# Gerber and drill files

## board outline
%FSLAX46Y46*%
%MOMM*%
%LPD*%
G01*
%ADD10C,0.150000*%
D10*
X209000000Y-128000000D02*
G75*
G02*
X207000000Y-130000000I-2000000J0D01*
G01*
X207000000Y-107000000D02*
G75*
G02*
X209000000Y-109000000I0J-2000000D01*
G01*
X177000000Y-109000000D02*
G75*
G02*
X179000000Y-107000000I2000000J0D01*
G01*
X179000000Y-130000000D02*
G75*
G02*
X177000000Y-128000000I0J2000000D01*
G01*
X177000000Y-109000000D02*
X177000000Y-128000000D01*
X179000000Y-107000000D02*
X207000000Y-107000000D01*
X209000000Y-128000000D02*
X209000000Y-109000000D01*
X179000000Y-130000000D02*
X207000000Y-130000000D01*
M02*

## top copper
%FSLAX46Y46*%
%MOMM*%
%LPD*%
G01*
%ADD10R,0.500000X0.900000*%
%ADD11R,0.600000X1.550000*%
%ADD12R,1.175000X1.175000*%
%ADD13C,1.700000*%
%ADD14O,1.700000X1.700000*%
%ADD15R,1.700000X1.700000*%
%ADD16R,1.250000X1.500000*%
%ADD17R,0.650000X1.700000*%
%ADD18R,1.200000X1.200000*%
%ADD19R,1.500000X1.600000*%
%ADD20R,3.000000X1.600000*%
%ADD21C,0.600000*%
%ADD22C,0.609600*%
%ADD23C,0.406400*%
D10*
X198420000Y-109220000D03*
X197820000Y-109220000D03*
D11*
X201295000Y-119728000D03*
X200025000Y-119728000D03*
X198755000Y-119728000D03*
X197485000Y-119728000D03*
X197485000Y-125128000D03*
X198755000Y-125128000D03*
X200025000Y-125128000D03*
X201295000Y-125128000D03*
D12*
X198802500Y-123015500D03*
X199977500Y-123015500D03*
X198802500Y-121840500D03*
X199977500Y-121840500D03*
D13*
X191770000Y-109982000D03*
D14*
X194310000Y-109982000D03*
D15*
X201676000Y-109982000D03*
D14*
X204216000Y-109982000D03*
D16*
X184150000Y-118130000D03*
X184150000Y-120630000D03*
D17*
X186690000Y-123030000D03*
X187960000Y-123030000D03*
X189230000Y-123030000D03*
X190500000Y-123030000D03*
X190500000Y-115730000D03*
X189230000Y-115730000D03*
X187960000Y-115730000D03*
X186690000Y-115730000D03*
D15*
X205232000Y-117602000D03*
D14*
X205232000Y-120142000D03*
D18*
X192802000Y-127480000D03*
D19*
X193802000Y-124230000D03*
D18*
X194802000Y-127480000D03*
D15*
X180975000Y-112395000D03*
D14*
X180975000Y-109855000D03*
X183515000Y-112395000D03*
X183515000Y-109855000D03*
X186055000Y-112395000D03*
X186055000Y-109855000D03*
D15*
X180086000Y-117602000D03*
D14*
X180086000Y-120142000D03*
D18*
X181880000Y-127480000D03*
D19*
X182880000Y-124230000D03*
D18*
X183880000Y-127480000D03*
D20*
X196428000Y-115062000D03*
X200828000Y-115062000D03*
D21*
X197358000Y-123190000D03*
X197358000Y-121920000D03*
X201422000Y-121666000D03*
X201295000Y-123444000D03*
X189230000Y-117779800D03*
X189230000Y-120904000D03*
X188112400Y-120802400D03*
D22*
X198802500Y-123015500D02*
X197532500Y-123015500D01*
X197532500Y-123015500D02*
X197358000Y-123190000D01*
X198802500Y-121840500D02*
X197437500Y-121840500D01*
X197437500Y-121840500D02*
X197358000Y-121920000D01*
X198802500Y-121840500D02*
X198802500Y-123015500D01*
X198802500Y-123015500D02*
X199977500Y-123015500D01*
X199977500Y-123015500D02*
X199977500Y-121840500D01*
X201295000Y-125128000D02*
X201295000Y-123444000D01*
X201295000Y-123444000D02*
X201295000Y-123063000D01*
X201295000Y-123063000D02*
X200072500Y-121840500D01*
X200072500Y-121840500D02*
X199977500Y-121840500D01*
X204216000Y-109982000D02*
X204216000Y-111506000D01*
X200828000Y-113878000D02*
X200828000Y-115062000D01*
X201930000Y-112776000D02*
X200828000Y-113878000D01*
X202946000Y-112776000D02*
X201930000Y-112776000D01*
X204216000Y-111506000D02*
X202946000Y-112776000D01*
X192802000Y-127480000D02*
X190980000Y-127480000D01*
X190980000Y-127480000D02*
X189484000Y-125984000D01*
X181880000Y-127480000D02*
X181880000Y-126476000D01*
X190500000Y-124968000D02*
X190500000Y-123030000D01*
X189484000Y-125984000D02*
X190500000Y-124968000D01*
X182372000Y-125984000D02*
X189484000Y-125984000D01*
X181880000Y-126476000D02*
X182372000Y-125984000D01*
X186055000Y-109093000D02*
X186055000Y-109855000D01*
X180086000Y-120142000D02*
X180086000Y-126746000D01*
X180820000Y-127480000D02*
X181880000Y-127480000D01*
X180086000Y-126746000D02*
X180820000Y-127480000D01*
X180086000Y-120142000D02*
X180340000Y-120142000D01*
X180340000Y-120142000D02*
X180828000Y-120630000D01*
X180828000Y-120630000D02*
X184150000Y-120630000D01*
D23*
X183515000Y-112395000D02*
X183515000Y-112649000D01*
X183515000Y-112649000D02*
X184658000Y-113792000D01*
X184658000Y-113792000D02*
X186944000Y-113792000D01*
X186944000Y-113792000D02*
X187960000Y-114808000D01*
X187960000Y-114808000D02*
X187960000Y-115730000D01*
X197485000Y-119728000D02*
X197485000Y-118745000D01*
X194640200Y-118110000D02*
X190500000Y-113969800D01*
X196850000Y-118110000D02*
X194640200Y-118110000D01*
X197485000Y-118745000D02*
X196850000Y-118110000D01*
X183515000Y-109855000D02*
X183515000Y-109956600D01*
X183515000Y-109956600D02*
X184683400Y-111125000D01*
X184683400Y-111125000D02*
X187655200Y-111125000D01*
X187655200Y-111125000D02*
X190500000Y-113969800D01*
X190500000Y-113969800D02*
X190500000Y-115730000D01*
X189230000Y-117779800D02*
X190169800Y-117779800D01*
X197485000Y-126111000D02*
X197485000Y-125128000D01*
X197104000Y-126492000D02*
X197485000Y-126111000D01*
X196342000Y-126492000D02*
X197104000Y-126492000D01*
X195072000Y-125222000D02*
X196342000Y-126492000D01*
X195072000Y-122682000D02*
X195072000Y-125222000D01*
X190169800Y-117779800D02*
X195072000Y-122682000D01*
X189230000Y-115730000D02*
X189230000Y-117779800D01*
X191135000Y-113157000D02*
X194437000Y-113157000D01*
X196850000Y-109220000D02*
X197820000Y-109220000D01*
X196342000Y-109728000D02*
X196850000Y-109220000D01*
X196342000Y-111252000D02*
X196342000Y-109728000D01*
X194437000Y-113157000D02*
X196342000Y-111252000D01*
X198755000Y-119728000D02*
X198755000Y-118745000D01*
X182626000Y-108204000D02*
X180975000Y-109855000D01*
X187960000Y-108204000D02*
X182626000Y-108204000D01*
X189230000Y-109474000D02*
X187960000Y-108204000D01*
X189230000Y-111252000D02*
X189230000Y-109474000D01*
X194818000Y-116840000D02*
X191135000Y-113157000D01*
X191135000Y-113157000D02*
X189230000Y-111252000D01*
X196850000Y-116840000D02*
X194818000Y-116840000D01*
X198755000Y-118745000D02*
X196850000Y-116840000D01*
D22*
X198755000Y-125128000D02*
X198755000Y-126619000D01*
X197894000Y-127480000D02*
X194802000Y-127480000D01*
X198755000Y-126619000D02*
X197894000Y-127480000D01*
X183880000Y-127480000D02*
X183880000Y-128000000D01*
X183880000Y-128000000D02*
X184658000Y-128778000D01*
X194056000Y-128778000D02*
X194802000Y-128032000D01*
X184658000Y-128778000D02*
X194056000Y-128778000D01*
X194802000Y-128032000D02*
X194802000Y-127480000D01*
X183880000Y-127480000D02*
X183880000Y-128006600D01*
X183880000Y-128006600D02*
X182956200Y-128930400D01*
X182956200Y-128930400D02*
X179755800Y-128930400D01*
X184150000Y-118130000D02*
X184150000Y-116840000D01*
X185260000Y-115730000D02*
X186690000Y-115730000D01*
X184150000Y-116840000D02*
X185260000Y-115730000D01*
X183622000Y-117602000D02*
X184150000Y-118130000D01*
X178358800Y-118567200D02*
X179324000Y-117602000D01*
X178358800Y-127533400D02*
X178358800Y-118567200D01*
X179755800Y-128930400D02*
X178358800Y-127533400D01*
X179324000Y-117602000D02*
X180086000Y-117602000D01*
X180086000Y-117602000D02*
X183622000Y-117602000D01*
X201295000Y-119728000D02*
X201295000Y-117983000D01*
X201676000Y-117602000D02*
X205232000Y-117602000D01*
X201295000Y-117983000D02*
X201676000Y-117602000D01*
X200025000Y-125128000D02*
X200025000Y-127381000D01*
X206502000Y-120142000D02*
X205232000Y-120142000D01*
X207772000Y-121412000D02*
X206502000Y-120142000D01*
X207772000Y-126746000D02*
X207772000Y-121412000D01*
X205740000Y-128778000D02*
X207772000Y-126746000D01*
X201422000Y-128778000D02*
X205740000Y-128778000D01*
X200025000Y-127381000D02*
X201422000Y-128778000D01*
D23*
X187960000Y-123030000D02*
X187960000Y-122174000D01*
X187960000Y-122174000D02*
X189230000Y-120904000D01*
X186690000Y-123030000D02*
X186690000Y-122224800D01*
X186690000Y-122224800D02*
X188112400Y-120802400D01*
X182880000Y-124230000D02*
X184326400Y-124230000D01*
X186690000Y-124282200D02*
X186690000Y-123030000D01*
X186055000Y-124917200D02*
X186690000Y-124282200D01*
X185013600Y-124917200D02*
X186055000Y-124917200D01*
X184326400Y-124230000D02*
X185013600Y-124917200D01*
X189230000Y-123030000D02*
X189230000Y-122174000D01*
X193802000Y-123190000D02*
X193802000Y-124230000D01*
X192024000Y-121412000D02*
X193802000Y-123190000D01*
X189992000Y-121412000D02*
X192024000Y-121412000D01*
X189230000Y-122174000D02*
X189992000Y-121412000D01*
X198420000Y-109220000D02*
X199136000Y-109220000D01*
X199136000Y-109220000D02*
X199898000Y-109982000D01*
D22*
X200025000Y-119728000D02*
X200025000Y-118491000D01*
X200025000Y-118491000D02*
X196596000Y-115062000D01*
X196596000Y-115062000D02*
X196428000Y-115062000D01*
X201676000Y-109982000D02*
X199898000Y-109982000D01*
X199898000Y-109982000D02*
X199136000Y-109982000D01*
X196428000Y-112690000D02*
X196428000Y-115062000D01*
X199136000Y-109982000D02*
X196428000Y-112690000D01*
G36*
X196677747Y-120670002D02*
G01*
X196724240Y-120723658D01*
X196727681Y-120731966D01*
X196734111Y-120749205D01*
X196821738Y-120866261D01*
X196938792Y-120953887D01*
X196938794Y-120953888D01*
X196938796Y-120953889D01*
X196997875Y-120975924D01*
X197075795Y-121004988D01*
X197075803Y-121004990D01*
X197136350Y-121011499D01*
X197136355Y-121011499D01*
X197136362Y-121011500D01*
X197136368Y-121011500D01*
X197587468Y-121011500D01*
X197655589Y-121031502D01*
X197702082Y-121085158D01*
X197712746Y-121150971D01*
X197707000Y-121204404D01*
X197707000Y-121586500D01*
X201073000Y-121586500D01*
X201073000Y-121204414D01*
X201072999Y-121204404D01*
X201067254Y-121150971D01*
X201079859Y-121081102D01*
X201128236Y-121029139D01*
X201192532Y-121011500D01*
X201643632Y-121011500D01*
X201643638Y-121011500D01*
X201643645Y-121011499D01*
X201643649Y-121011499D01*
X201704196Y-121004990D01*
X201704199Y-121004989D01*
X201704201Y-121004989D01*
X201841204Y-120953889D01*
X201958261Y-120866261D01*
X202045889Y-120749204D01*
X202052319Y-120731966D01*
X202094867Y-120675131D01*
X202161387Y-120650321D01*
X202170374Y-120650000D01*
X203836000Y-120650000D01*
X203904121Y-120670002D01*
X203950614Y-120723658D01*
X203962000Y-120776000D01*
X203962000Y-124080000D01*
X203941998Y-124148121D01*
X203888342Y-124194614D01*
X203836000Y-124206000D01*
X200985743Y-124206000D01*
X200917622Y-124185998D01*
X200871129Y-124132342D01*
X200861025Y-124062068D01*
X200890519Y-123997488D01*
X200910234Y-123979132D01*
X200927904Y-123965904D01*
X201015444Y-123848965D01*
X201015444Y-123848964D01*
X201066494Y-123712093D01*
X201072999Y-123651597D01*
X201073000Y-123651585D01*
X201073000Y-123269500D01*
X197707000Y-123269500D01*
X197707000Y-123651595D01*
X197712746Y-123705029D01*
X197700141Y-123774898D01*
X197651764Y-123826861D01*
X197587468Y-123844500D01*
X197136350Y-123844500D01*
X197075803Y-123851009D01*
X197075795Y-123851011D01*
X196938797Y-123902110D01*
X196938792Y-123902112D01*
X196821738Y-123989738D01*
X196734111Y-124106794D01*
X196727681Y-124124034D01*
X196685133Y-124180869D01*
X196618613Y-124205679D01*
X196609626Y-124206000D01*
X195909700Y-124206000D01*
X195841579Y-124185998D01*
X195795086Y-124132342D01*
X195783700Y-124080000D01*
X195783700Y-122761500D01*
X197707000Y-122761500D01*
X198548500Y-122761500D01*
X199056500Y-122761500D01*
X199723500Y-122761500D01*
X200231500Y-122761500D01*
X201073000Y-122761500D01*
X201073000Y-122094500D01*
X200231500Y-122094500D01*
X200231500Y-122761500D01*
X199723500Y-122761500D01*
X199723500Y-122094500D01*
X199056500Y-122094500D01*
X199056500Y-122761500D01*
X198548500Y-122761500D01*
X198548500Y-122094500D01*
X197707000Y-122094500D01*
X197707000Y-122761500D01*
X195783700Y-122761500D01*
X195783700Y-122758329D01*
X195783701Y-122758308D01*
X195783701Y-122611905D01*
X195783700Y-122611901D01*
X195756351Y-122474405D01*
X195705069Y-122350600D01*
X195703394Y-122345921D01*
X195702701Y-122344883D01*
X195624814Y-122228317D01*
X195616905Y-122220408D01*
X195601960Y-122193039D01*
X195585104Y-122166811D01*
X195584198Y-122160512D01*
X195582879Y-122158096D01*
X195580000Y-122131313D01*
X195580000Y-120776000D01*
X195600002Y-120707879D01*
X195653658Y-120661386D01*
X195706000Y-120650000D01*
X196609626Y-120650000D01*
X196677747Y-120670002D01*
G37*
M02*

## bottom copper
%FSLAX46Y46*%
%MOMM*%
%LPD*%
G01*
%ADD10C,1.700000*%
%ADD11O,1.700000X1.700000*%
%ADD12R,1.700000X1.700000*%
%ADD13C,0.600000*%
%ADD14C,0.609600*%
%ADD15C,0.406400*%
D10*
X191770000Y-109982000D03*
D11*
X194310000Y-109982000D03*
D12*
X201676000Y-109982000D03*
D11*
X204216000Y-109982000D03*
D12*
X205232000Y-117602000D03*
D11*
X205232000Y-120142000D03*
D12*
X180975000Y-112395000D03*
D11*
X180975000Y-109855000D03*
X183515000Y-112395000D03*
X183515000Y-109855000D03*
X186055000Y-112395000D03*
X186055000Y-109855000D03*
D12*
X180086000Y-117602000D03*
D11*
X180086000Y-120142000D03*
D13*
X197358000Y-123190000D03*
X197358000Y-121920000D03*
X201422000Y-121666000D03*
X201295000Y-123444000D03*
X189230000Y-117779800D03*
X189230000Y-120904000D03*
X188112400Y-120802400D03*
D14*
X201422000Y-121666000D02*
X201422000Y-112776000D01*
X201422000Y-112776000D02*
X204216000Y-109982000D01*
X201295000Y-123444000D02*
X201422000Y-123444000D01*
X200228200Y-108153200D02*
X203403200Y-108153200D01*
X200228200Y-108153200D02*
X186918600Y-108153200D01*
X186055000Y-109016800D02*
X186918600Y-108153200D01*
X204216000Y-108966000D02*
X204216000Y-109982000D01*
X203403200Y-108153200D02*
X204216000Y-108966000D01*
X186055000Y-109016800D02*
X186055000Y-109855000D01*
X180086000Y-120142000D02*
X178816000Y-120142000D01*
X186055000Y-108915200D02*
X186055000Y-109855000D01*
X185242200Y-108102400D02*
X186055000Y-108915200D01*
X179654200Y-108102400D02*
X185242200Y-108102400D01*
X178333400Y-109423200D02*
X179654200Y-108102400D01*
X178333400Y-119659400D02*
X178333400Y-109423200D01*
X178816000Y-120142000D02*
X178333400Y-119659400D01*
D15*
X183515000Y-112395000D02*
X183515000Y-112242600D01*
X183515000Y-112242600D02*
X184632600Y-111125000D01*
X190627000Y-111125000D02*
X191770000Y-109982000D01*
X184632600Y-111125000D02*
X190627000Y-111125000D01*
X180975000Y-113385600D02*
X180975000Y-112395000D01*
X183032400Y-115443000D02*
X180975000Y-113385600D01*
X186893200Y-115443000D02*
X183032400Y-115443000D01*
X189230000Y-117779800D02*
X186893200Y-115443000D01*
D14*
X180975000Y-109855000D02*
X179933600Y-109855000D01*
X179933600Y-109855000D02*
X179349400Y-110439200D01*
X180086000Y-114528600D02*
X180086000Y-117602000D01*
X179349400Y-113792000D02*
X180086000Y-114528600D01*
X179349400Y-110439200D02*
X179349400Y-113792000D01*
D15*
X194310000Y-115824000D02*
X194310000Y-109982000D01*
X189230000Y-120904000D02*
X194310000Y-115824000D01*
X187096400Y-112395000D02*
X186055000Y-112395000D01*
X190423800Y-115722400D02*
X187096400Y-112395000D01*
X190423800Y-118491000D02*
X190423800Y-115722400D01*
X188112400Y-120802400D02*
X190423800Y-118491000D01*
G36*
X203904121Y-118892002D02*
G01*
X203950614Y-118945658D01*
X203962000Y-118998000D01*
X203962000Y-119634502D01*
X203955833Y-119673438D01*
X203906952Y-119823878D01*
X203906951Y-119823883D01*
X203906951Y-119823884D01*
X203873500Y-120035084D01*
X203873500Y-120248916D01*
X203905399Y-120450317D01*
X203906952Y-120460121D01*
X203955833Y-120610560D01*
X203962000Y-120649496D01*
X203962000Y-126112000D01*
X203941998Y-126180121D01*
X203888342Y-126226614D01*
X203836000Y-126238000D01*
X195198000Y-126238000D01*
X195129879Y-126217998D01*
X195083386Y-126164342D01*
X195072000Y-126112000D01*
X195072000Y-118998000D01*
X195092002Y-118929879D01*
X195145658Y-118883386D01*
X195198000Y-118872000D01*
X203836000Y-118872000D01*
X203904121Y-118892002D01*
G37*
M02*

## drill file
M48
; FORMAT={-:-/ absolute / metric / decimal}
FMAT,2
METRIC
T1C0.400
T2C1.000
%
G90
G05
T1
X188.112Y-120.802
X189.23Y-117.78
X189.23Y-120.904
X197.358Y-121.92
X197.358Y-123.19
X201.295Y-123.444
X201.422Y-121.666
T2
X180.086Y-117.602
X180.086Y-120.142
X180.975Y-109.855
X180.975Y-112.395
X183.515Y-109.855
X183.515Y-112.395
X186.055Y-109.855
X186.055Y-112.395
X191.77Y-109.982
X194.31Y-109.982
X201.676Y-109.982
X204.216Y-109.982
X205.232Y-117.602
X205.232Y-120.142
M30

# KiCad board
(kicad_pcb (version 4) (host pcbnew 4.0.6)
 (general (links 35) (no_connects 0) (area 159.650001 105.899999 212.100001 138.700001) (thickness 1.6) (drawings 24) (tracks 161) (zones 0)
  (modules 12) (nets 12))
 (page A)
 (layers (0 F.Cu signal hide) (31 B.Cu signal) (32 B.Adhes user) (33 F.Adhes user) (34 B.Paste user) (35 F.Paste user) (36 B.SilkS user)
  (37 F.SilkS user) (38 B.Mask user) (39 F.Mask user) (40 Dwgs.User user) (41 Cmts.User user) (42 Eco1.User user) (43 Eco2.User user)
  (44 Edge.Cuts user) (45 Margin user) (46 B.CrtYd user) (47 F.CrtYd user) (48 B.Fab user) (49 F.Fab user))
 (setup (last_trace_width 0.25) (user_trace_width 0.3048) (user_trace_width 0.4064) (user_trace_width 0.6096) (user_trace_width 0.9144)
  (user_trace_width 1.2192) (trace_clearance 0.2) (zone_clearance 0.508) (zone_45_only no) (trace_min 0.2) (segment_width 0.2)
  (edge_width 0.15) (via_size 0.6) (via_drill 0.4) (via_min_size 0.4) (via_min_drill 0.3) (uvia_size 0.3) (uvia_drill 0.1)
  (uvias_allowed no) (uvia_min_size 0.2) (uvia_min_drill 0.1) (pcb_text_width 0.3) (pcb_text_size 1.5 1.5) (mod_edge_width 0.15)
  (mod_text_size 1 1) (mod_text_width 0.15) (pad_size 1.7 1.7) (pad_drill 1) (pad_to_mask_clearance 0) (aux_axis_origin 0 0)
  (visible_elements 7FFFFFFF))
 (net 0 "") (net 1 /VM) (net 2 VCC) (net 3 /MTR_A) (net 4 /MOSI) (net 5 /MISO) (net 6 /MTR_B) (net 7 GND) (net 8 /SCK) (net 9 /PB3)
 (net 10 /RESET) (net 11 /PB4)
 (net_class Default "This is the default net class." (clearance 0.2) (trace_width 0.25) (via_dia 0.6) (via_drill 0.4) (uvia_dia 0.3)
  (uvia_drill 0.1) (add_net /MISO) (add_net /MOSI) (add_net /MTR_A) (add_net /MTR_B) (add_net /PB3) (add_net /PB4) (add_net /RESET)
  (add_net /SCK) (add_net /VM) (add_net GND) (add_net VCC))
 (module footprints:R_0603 (layer F.Cu) (at 198.12 109.22 180)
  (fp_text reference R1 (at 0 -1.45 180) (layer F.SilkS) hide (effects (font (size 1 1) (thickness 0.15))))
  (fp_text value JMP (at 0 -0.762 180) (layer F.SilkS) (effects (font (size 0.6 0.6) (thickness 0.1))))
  (pad 1 smd rect (at -0.3 0 180) (size 0.5 0.9) (layers F.Cu F.Paste F.Mask) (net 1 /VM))
  (pad 2 smd rect (at 0.3 0 180) (size 0.5 0.9) (layers F.Cu F.Paste F.Mask) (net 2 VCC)))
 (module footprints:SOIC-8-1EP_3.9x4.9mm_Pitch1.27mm (layer F.Cu) (at 199.39 122.428 270)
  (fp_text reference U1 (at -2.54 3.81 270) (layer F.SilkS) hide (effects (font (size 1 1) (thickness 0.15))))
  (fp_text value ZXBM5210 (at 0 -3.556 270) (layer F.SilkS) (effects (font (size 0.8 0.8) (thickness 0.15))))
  (pad 1 smd rect (at -2.7 -1.905 270) (size 1.55 0.6) (layers F.Cu F.Paste F.Mask) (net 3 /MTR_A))
  (pad 2 smd rect (at -2.7 -0.635 270) (size 1.55 0.6) (layers F.Cu F.Paste F.Mask) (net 1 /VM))
  (pad 3 smd rect (at -2.7 0.635 270) (size 1.55 0.6) (layers F.Cu F.Paste F.Mask) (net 2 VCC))
  (pad 4 smd rect (at -2.7 1.905 270) (size 1.55 0.6) (layers F.Cu F.Paste F.Mask) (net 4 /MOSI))
  (pad 5 smd rect (at 2.7 1.905 270) (size 1.55 0.6) (layers F.Cu F.Paste F.Mask) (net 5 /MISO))
  (pad 6 smd rect (at 2.7 0.635 270) (size 1.55 0.6) (layers F.Cu F.Paste F.Mask) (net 2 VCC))
  (pad 7 smd rect (at 2.7 -0.635 270) (size 1.55 0.6) (layers F.Cu F.Paste F.Mask) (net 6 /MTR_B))
  (pad 8 smd rect (at 2.7 -1.905 270) (size 1.55 0.6) (layers F.Cu F.Paste F.Mask) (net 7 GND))
  (pad 8 smd rect (at 0.5875 0.5875 270) (size 1.175 1.175) (layers F.Cu F.Paste F.Mask) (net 7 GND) (solder_paste_margin_ratio -0.2))
  (pad 8 smd rect (at 0.5875 -0.5875 270) (size 1.175 1.175) (layers F.Cu F.Paste F.Mask) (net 7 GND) (solder_paste_margin_ratio -0.2))
  (pad 8 smd rect (at -0.5875 0.5875 270) (size 1.175 1.175) (layers F.Cu F.Paste F.Mask) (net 7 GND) (solder_paste_margin_ratio -0.2))
  (pad 8 smd rect (at -0.5875 -0.5875 270) (size 1.175 1.175) (layers F.Cu F.Paste F.Mask) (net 7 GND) (solder_paste_margin_ratio -0.2)))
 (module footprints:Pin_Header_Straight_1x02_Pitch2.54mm (layer F.Cu) (at 191.77 109.982 90)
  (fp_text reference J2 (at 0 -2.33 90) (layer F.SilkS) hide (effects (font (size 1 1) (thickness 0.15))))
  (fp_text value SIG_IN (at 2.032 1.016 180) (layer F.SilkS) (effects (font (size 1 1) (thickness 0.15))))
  (pad 1 thru_hole circle (at 0 0 90) (size 1.7 1.7) (drill 1) (layers *.Cu *.Mask) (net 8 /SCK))
  (pad 2 thru_hole oval (at 0 2.54 90) (size 1.7 1.7) (drill 1) (layers *.Cu *.Mask) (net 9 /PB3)))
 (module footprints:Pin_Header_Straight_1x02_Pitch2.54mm (layer F.Cu) (at 201.676 109.982 90)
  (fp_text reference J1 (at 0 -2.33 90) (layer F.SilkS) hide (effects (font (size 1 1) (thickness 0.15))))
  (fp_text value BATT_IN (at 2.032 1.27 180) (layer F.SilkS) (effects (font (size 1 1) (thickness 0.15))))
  (pad 1 thru_hole rect (at 0 0 90) (size 1.7 1.7) (drill 1) (layers *.Cu *.Mask) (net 1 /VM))
  (pad 2 thru_hole oval (at 0 2.54 90) (size 1.7 1.7) (drill 1) (layers *.Cu *.Mask) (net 7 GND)))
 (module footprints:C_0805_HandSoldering (layer F.Cu) (at 184.15 119.38 270)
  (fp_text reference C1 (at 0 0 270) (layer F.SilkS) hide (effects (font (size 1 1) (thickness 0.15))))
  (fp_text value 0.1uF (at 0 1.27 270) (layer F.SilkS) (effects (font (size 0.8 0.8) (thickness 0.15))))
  (pad 1 smd rect (at -1.25 0 270) (size 1.5 1.25) (layers F.Cu F.Paste F.Mask) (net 2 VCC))
  (pad 2 smd rect (at 1.25 0 270) (size 1.5 1.25) (layers F.Cu F.Paste F.Mask) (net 7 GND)))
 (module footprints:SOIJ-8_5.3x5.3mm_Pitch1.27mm (layer F.Cu) (at 188.595 119.38 90)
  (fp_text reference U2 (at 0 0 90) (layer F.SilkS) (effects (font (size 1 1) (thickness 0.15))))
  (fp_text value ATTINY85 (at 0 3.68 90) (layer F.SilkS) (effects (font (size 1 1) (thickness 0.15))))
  (pad 1 smd rect (at -3.65 -1.905 90) (size 1.7 0.65) (layers F.Cu F.Paste F.Mask) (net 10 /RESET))
  (pad 2 smd rect (at -3.65 -0.635 90) (size 1.7 0.65) (layers F.Cu F.Paste F.Mask) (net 9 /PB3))
  (pad 3 smd rect (at -3.65 0.635 90) (size 1.7 0.65) (layers F.Cu F.Paste F.Mask) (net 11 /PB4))
  (pad 4 smd rect (at -3.65 1.905 90) (size 1.7 0.65) (layers F.Cu F.Paste F.Mask) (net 7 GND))
  (pad 5 smd rect (at 3.65 1.905 90) (size 1.7 0.65) (layers F.Cu F.Paste F.Mask) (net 4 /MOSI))
  (pad 6 smd rect (at 3.65 0.635 90) (size 1.7 0.65) (layers F.Cu F.Paste F.Mask) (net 5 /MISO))
  (pad 7 smd rect (at 3.65 -0.635 90) (size 1.7 0.65) (layers F.Cu F.Paste F.Mask) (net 8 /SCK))
  (pad 8 smd rect (at 3.65 -1.905 90) (size 1.7 0.65) (layers F.Cu F.Paste F.Mask) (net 2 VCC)))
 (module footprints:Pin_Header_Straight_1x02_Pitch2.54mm (layer F.Cu) (at 205.232 117.602)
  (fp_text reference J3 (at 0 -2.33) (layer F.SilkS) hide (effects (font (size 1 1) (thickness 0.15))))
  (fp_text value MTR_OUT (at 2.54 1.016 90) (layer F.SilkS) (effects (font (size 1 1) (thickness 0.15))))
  (pad 1 thru_hole rect (at 0 0) (size 1.7 1.7) (drill 1) (layers *.Cu *.Mask) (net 3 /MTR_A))
  (pad 2 thru_hole oval (at 0 2.54) (size 1.7 1.7) (drill 1) (layers *.Cu *.Mask) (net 6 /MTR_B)))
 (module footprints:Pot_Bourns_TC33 (layer F.Cu) (at 193.802 125.73)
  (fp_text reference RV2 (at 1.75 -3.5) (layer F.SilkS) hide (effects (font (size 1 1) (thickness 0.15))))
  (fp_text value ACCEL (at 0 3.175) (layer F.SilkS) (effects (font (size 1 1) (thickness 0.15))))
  (pad 1 smd rect (at -1 1.75) (size 1.2 1.2) (layers F.Cu F.Mask) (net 7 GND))
  (pad 2 smd rect (at 0 -1.5) (size 1.5 1.6) (layers F.Cu F.Mask) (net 11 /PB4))
  (pad 3 smd rect (at 1 1.75) (size 1.2 1.2) (layers F.Cu F.Mask) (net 2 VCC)))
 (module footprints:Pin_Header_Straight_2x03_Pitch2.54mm (layer F.Cu) (at 180.975 112.395 90)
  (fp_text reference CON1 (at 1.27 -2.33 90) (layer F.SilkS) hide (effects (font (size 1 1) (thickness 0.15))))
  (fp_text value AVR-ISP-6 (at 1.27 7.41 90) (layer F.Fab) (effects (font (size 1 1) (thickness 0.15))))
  (pad 1 thru_hole rect (at 0 0 90) (size 1.7 1.7) (drill 1) (layers *.Cu *.Mask) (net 5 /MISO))
  (pad 2 thru_hole oval (at 2.54 0 90) (size 1.7 1.7) (drill 1) (layers *.Cu *.Mask) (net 2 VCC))
  (pad 3 thru_hole oval (at 0 2.54 90) (size 1.7 1.7) (drill 1) (layers *.Cu *.Mask) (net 8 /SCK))
  (pad 4 thru_hole oval (at 2.54 2.54 90) (size 1.7 1.7) (drill 1) (layers *.Cu *.Mask) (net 4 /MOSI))
  (pad 5 thru_hole oval (at 0 5.08 90) (size 1.7 1.7) (drill 1) (layers *.Cu *.Mask) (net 10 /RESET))
  (pad 6 thru_hole oval (at 2.54 5.08 90) (size 1.7 1.7) (drill 1) (layers *.Cu *.Mask) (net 7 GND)))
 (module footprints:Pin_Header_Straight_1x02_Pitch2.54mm (layer F.Cu) (at 180.086 117.602)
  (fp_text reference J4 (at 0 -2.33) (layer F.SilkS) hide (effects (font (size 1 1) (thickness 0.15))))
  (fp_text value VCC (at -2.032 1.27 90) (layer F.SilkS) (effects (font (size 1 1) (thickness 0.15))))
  (pad 1 thru_hole rect (at 0 0) (size 1.7 1.7) (drill 1) (layers *.Cu *.Mask) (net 2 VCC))
  (pad 2 thru_hole oval (at 0 2.54) (size 1.7 1.7) (drill 1) (layers *.Cu *.Mask) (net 7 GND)))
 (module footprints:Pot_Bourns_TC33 (layer F.Cu) (at 182.88 125.73)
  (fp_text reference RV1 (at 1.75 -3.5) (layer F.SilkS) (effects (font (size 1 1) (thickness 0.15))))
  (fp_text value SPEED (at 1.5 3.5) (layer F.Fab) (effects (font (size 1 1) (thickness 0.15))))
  (pad 1 smd rect (at -1 1.75) (size 1.2 1.2) (layers F.Cu F.Mask) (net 7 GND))
  (pad 2 smd rect (at 0 -1.5) (size 1.5 1.6) (layers F.Cu F.Mask) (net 10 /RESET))
  (pad 3 smd rect (at 1 1.75) (size 1.2 1.2) (layers F.Cu F.Mask) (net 2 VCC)))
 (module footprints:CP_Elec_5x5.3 (layer F.Cu) (at 198.628 115.062)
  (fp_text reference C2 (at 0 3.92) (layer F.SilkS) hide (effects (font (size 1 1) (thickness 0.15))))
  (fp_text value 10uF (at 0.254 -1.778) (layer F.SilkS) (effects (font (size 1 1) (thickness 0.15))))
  (pad 1 smd rect (at -2.2 0 180) (size 3 1.6) (layers F.Cu F.Paste F.Mask) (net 1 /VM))
  (pad 2 smd rect (at 2.2 0 180) (size 3 1.6) (layers F.Cu F.Paste F.Mask) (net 7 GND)))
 (gr_arc (start 207 128) (end 209 128) (angle 90) (layer Edge.Cuts) (width 0.15))
 (gr_arc (start 207 109) (end 207 107) (angle 90) (layer Edge.Cuts) (width 0.15))
 (gr_arc (start 179 109) (end 177 109) (angle 90) (layer Edge.Cuts) (width 0.15))
 (gr_arc (start 179 128) (end 179 130) (angle 90) (layer Edge.Cuts) (width 0.15))
 (gr_line (start 177 109) (end 177 128) (angle 90) (layer Edge.Cuts) (width 0.15))
 (gr_line (start 179 107) (end 207 107) (angle 90) (layer Edge.Cuts) (width 0.15))
 (gr_line (start 209 128) (end 209 109) (angle 90) (layer Edge.Cuts) (width 0.15))
 (gr_line (start 179 130) (end 207 130) (angle 90) (layer Edge.Cuts) (width 0.15))
 (segment (start 198.8025 123.0155) (end 197.5325 123.0155) (width 0.6096) (layer F.Cu) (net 7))
 (via (at 197.358 123.19) (size 0.6) (drill 0.4) (layers F.Cu B.Cu) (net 7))
 (segment (start 197.5325 123.0155) (end 197.358 123.19) (width 0.6096) (layer F.Cu) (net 7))
 (segment (start 198.8025 121.8405) (end 197.4375 121.8405) (width 0.6096) (layer F.Cu) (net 7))
 (via (at 197.358 121.92) (size 0.6) (drill 0.4) (layers F.Cu B.Cu) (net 7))
 (segment (start 197.4375 121.8405) (end 197.358 121.92) (width 0.6096) (layer F.Cu) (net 7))
 (segment (start 201.422 121.666) (end 201.422 112.776) (width 0.6096) (layer B.Cu) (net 7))
 (via (at 201.422 121.666) (size 0.6) (drill 0.4) (layers F.Cu B.Cu) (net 7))
 (segment (start 201.422 112.776) (end 204.216 109.982) (width 0.6096) (layer B.Cu) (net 7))
 (via (at 201.295 123.444) (size 0.6) (drill 0.4) (layers F.Cu B.Cu) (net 7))
 (segment (start 201.295 123.444) (end 201.422 123.444) (width 0.6096) (layer B.Cu) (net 7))
 (segment (start 198.8025 121.8405) (end 198.8025 123.0155) (width 0.6096) (layer F.Cu) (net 7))
 (segment (start 198.8025 123.0155) (end 199.9775 123.0155) (width 0.6096) (layer F.Cu) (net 7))
 (segment (start 199.9775 123.0155) (end 199.9775 121.8405) (width 0.6096) (layer F.Cu) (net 7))
 (segment (start 201.295 125.128) (end 201.295 123.444) (width 0.6096) (layer F.Cu) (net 7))
 (segment (start 201.295 123.444) (end 201.295 123.063) (width 0.6096) (layer F.Cu) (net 7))
 (segment (start 201.295 123.063) (end 200.0725 121.8405) (width 0.6096) (layer F.Cu) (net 7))
 (segment (start 200.0725 121.8405) (end 199.9775 121.8405) (width 0.6096) (layer F.Cu) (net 7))
 (segment (start 204.216 109.982) (end 204.216 111.506) (width 0.6096) (layer F.Cu) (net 7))
 (segment (start 200.828 113.878) (end 200.828 115.062) (width 0.6096) (layer F.Cu) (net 7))
 (segment (start 201.93 112.776) (end 200.828 113.878) (width 0.6096) (layer F.Cu) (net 7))
 (segment (start 202.946 112.776) (end 201.93 112.776) (width 0.6096) (layer F.Cu) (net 7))
 (segment (start 204.216 111.506) (end 202.946 112.776) (width 0.6096) (layer F.Cu) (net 7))
 (segment (start 192.802 127.48) (end 190.98 127.48) (width 0.6096) (layer F.Cu) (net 7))
 (segment (start 190.98 127.48) (end 189.484 125.984) (width 0.6096) (layer F.Cu) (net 7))
 (segment (start 200.2282 108.1532) (end 203.4032 108.1532) (width 0.6096) (layer B.Cu) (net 7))
 (segment (start 200.2282 108.1532) (end 186.9186 108.1532) (width 0.6096) (layer B.Cu) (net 7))
 (segment (start 186.055 109.0168) (end 186.9186 108.1532) (width 0.6096) (layer B.Cu) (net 7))
 (segment (start 204.216 108.966) (end 204.216 109.982) (width 0.6096) (layer B.Cu) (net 7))
 (segment (start 203.4032 108.1532) (end 204.216 108.966) (width 0.6096) (layer B.Cu) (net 7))
 (segment (start 186.055 109.0168) (end 186.055 109.855) (width 0.6096) (layer B.Cu) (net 7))
 (segment (start 180.086 120.142) (end 178.816 120.142) (width 0.6096) (layer B.Cu) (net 7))
 (segment (start 186.055 108.9152) (end 186.055 109.855) (width 0.6096) (layer B.Cu) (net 7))
 (segment (start 185.2422 108.1024) (end 186.055 108.9152) (width 0.6096) (layer B.Cu) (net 7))
 (segment (start 179.6542 108.1024) (end 185.2422 108.1024) (width 0.6096) (layer B.Cu) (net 7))
 (segment (start 178.3334 109.4232) (end 179.6542 108.1024) (width 0.6096) (layer B.Cu) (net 7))
 (segment (start 178.3334 119.6594) (end 178.3334 109.4232) (width 0.6096) (layer B.Cu) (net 7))
 (segment (start 178.816 120.142) (end 178.3334 119.6594) (width 0.6096) (layer B.Cu) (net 7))
 (segment (start 181.88 127.48) (end 181.88 126.476) (width 0.6096) (layer F.Cu) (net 7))
 (segment (start 190.5 124.968) (end 190.5 123.03) (width 0.6096) (layer F.Cu) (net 7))
 (segment (start 189.484 125.984) (end 190.5 124.968) (width 0.6096) (layer F.Cu) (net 7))
 (segment (start 182.372 125.984) (end 189.484 125.984) (width 0.6096) (layer F.Cu) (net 7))
 (segment (start 181.88 126.476) (end 182.372 125.984) (width 0.6096) (layer F.Cu) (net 7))
 (segment (start 186.055 109.093) (end 186.055 109.855) (width 0.6096) (layer F.Cu) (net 7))
 (segment (start 180.086 120.142) (end 180.086 126.746) (width 0.6096) (layer F.Cu) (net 7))
 (segment (start 180.82 127.48) (end 181.88 127.48) (width 0.6096) (layer F.Cu) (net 7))
 (segment (start 180.086 126.746) (end 180.82 127.48) (width 0.6096) (layer F.Cu) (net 7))
 (segment (start 180.086 120.142) (end 180.34 120.142) (width 0.6096) (layer F.Cu) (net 7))
 (segment (start 180.34 120.142) (end 180.828 120.63) (width 0.6096) (layer F.Cu) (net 7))
 (segment (start 180.828 120.63) (end 184.15 120.63) (width 0.6096) (layer F.Cu) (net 7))
 (segment (start 183.515 112.395) (end 183.515 112.2426) (width 0.4064) (layer B.Cu) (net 8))
 (segment (start 183.515 112.2426) (end 184.6326 111.125) (width 0.4064) (layer B.Cu) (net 8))
 (segment (start 190.627 111.125) (end 191.77 109.982) (width 0.4064) (layer B.Cu) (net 8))
 (segment (start 184.6326 111.125) (end 190.627 111.125) (width 0.4064) (layer B.Cu) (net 8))
 (segment (start 183.515 112.395) (end 183.515 112.649) (width 0.4064) (layer F.Cu) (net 8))
 (segment (start 183.515 112.649) (end 184.658 113.792) (width 0.4064) (layer F.Cu) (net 8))
 (segment (start 184.658 113.792) (end 186.944 113.792) (width 0.4064) (layer F.Cu) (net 8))
 (segment (start 186.944 113.792) (end 187.96 114.808) (width 0.4064) (layer F.Cu) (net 8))
 (segment (start 187.96 114.808) (end 187.96 115.73) (width 0.4064) (layer F.Cu) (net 8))
 (segment (start 197.485 119.728) (end 197.485 118.745) (width 0.4064) (layer F.Cu) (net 4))
 (segment (start 194.6402 118.11) (end 190.5 113.9698) (width 0.4064) (layer F.Cu) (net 4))
 (segment (start 196.85 118.11) (end 194.6402 118.11) (width 0.4064) (layer F.Cu) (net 4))
 (segment (start 197.485 118.745) (end 196.85 118.11) (width 0.4064) (layer F.Cu) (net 4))
 (segment (start 183.515 109.855) (end 183.515 109.9566) (width 0.4064) (layer F.Cu) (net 4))
 (segment (start 183.515 109.9566) (end 184.6834 111.125) (width 0.4064) (layer F.Cu) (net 4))
 (segment (start 184.6834 111.125) (end 187.6552 111.125) (width 0.4064) (layer F.Cu) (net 4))
 (segment (start 187.6552 111.125) (end 190.5 113.9698) (width 0.4064) (layer F.Cu) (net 4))
 (segment (start 190.5 113.9698) (end 190.5 115.73) (width 0.4064) (layer F.Cu) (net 4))
 (segment (start 189.23 117.7798) (end 190.1698 117.7798) (width 0.4064) (layer F.Cu) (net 5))
 (segment (start 197.485 126.111) (end 197.485 125.128) (width 0.4064) (layer F.Cu) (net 5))
 (segment (start 197.104 126.492) (end 197.485 126.111) (width 0.4064) (layer F.Cu) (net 5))
 (segment (start 196.342 126.492) (end 197.104 126.492) (width 0.4064) (layer F.Cu) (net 5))
 (segment (start 195.072 125.222) (end 196.342 126.492) (width 0.4064) (layer F.Cu) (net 5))
 (segment (start 195.072 122.682) (end 195.072 125.222) (width 0.4064) (layer F.Cu) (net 5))
 (segment (start 190.1698 117.7798) (end 195.072 122.682) (width 0.4064) (layer F.Cu) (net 5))
 (segment (start 189.23 115.73) (end 189.23 117.7798) (width 0.4064) (layer F.Cu) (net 5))
 (via (at 189.23 117.7798) (size 0.6) (drill 0.4) (layers F.Cu B.Cu) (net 5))
 (segment (start 180.975 113.3856) (end 180.975 112.395) (width 0.4064) (layer B.Cu) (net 5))
 (segment (start 183.0324 115.443) (end 180.975 113.3856) (width 0.4064) (layer B.Cu) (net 5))
 (segment (start 186.8932 115.443) (end 183.0324 115.443) (width 0.4064) (layer B.Cu) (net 5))
 (segment (start 189.23 117.7798) (end 186.8932 115.443) (width 0.4064) (layer B.Cu) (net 5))
 (segment (start 191.135 113.157) (end 194.437 113.157) (width 0.4064) (layer F.Cu) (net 2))
 (segment (start 196.85 109.22) (end 197.82 109.22) (width 0.4064) (layer F.Cu) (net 2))
 (segment (start 196.342 109.728) (end 196.85 109.22) (width 0.4064) (layer F.Cu) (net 2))
 (segment (start 196.342 111.252) (end 196.342 109.728) (width 0.4064) (layer F.Cu) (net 2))
 (segment (start 194.437 113.157) (end 196.342 111.252) (width 0.4064) (layer F.Cu) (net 2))
 (segment (start 198.755 119.728) (end 198.755 118.745) (width 0.4064) (layer F.Cu) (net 2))
 (segment (start 182.626 108.204) (end 180.975 109.855) (width 0.4064) (layer F.Cu) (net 2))
 (segment (start 187.96 108.204) (end 182.626 108.204) (width 0.4064) (layer F.Cu) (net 2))
 (segment (start 189.23 109.474) (end 187.96 108.204) (width 0.4064) (layer F.Cu) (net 2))
 (segment (start 189.23 111.252) (end 189.23 109.474) (width 0.4064) (layer F.Cu) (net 2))
 (segment (start 194.818 116.84) (end 191.135 113.157) (width 0.4064) (layer F.Cu) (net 2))
 (segment (start 191.135 113.157) (end 189.23 111.252) (width 0.4064) (layer F.Cu) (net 2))
 (segment (start 196.85 116.84) (end 194.818 116.84) (width 0.4064) (layer F.Cu) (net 2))
 (segment (start 198.755 118.745) (end 196.85 116.84) (width 0.4064) (layer F.Cu) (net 2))
 (segment (start 198.755 125.128) (end 198.755 126.619) (width 0.6096) (layer F.Cu) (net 2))
 (segment (start 197.894 127.48) (end 194.802 127.48) (width 0.6096) (layer F.Cu) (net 2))
 (segment (start 198.755 126.619) (end 197.894 127.48) (width 0.6096) (layer F.Cu) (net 2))
 (segment (start 183.88 127.48) (end 183.88 128) (width 0.6096) (layer F.Cu) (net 2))
 (segment (start 183.88 128) (end 184.658 128.778) (width 0.6096) (layer F.Cu) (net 2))
 (segment (start 194.056 128.778) (end 194.802 128.032) (width 0.6096) (layer F.Cu) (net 2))
 (segment (start 184.658 128.778) (end 194.056 128.778) (width 0.6096) (layer F.Cu) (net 2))
 (segment (start 194.802 128.032) (end 194.802 127.48) (width 0.6096) (layer F.Cu) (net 2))
 (segment (start 183.88 127.48) (end 183.88 128.0066) (width 0.6096) (layer F.Cu) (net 2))
 (segment (start 183.88 128.0066) (end 182.9562 128.9304) (width 0.6096) (layer F.Cu) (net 2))
 (segment (start 182.9562 128.9304) (end 179.7558 128.9304) (width 0.6096) (layer F.Cu) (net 2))
 (segment (start 180.975 109.855) (end 179.9336 109.855) (width 0.6096) (layer B.Cu) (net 2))
 (segment (start 179.9336 109.855) (end 179.3494 110.4392) (width 0.6096) (layer B.Cu) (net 2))
 (segment (start 184.15 118.13) (end 184.15 116.84) (width 0.6096) (layer F.Cu) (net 2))
 (segment (start 185.26 115.73) (end 186.69 115.73) (width 0.6096) (layer F.Cu) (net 2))
 (segment (start 184.15 116.84) (end 185.26 115.73) (width 0.6096) (layer F.Cu) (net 2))
 (segment (start 183.622 117.602) (end 184.15 118.13) (width 0.6096) (layer F.Cu) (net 2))
 (segment (start 178.3588 118.5672) (end 179.324 117.602) (width 0.6096) (layer F.Cu) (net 2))
 (segment (start 178.3588 127.5334) (end 178.3588 118.5672) (width 0.6096) (layer F.Cu) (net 2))
 (segment (start 179.7558 128.9304) (end 178.3588 127.5334) (width 0.6096) (layer F.Cu) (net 2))
 (segment (start 179.324 117.602) (end 180.086 117.602) (width 0.6096) (layer F.Cu) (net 2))
 (segment (start 180.086 114.5286) (end 180.086 117.602) (width 0.6096) (layer B.Cu) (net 2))
 (segment (start 179.3494 113.792) (end 180.086 114.5286) (width 0.6096) (layer B.Cu) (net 2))
 (segment (start 179.3494 110.4392) (end 179.3494 113.792) (width 0.6096) (layer B.Cu) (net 2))
 (segment (start 180.086 117.602) (end 183.622 117.602) (width 0.6096) (layer F.Cu) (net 2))
 (segment (start 201.295 119.728) (end 201.295 117.983) (width 0.6096) (layer F.Cu) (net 3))
 (segment (start 201.676 117.602) (end 205.232 117.602) (width 0.6096) (layer F.Cu) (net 3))
 (segment (start 201.295 117.983) (end 201.676 117.602) (width 0.6096) (layer F.Cu) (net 3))
 (segment (start 200.025 125.128) (end 200.025 127.381) (width 0.6096) (layer F.Cu) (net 6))
 (segment (start 206.502 120.142) (end 205.232 120.142) (width 0.6096) (layer F.Cu) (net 6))
 (segment (start 207.772 121.412) (end 206.502 120.142) (width 0.6096) (layer F.Cu) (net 6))
 (segment (start 207.772 126.746) (end 207.772 121.412) (width 0.6096) (layer F.Cu) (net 6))
 (segment (start 205.74 128.778) (end 207.772 126.746) (width 0.6096) (layer F.Cu) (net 6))
 (segment (start 201.422 128.778) (end 205.74 128.778) (width 0.6096) (layer F.Cu) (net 6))
 (segment (start 200.025 127.381) (end 201.422 128.778) (width 0.6096) (layer F.Cu) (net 6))
 (segment (start 187.96 123.03) (end 187.96 122.174) (width 0.4064) (layer F.Cu) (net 9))
 (segment (start 194.31 115.824) (end 194.31 109.982) (width 0.4064) (layer B.Cu) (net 9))
 (segment (start 189.23 120.904) (end 194.31 115.824) (width 0.4064) (layer B.Cu) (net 9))
 (via (at 189.23 120.904) (size 0.6) (drill 0.4) (layers F.Cu B.Cu) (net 9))
 (segment (start 187.96 122.174) (end 189.23 120.904) (width 0.4064) (layer F.Cu) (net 9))
 (segment (start 186.69 123.03) (end 186.69 122.2248) (width 0.4064) (layer F.Cu) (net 10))
 (segment (start 186.69 122.2248) (end 188.1124 120.8024) (width 0.4064) (layer F.Cu) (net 10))
 (segment (start 187.0964 112.395) (end 186.055 112.395) (width 0.4064) (layer B.Cu) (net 10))
 (segment (start 190.4238 115.7224) (end 187.0964 112.395) (width 0.4064) (layer B.Cu) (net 10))
 (segment (start 190.4238 118.491) (end 190.4238 115.7224) (width 0.4064) (layer B.Cu) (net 10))
 (segment (start 188.1124 120.8024) (end 190.4238 118.491) (width 0.4064) (layer B.Cu) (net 10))
 (via (at 188.1124 120.8024) (size 0.6) (drill 0.4) (layers F.Cu B.Cu) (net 10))
 (segment (start 182.88 124.23) (end 184.3264 124.23) (width 0.4064) (layer F.Cu) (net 10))
 (segment (start 186.69 124.2822) (end 186.69 123.03) (width 0.4064) (layer F.Cu) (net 10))
 (segment (start 186.055 124.9172) (end 186.69 124.2822) (width 0.4064) (layer F.Cu) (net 10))
 (segment (start 185.0136 124.9172) (end 186.055 124.9172) (width 0.4064) (layer F.Cu) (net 10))
 (segment (start 184.3264 124.23) (end 185.0136 124.9172) (width 0.4064) (layer F.Cu) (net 10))
 (segment (start 189.23 123.03) (end 189.23 122.174) (width 0.4064) (layer F.Cu) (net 11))
 (segment (start 193.802 123.19) (end 193.802 124.23) (width 0.4064) (layer F.Cu) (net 11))
 (segment (start 192.024 121.412) (end 193.802 123.19) (width 0.4064) (layer F.Cu) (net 11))
 (segment (start 189.992 121.412) (end 192.024 121.412) (width 0.4064) (layer F.Cu) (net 11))
 (segment (start 189.23 122.174) (end 189.992 121.412) (width 0.4064) (layer F.Cu) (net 11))
 (segment (start 198.42 109.22) (end 199.136 109.22) (width 0.4064) (layer F.Cu) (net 1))
 (segment (start 199.136 109.22) (end 199.898 109.982) (width 0.4064) (layer F.Cu) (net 1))
 (segment (start 200.025 119.728) (end 200.025 118.491) (width 0.6096) (layer F.Cu) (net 1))
 (segment (start 200.025 118.491) (end 196.596 115.062) (width 0.6096) (layer F.Cu) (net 1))
 (segment (start 196.596 115.062) (end 196.428 115.062) (width 0.6096) (layer F.Cu) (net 1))
 (segment (start 201.676 109.982) (end 199.898 109.982) (width 0.6096) (layer F.Cu) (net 1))
 (segment (start 199.898 109.982) (end 199.136 109.982) (width 0.6096) (layer F.Cu) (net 1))
 (segment (start 196.428 112.69) (end 196.428 115.062) (width 0.6096) (layer F.Cu) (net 1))
 (segment (start 199.136 109.982) (end 196.428 112.69) (width 0.6096) (layer F.Cu) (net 1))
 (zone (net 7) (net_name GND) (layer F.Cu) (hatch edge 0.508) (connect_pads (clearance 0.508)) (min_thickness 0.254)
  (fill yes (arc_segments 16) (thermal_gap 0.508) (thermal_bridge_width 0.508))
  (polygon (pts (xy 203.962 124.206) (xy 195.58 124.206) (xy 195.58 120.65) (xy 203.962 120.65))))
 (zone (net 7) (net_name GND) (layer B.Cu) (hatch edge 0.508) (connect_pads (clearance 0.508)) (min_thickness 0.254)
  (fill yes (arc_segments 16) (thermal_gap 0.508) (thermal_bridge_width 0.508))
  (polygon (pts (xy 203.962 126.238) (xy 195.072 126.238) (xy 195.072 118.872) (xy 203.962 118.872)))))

